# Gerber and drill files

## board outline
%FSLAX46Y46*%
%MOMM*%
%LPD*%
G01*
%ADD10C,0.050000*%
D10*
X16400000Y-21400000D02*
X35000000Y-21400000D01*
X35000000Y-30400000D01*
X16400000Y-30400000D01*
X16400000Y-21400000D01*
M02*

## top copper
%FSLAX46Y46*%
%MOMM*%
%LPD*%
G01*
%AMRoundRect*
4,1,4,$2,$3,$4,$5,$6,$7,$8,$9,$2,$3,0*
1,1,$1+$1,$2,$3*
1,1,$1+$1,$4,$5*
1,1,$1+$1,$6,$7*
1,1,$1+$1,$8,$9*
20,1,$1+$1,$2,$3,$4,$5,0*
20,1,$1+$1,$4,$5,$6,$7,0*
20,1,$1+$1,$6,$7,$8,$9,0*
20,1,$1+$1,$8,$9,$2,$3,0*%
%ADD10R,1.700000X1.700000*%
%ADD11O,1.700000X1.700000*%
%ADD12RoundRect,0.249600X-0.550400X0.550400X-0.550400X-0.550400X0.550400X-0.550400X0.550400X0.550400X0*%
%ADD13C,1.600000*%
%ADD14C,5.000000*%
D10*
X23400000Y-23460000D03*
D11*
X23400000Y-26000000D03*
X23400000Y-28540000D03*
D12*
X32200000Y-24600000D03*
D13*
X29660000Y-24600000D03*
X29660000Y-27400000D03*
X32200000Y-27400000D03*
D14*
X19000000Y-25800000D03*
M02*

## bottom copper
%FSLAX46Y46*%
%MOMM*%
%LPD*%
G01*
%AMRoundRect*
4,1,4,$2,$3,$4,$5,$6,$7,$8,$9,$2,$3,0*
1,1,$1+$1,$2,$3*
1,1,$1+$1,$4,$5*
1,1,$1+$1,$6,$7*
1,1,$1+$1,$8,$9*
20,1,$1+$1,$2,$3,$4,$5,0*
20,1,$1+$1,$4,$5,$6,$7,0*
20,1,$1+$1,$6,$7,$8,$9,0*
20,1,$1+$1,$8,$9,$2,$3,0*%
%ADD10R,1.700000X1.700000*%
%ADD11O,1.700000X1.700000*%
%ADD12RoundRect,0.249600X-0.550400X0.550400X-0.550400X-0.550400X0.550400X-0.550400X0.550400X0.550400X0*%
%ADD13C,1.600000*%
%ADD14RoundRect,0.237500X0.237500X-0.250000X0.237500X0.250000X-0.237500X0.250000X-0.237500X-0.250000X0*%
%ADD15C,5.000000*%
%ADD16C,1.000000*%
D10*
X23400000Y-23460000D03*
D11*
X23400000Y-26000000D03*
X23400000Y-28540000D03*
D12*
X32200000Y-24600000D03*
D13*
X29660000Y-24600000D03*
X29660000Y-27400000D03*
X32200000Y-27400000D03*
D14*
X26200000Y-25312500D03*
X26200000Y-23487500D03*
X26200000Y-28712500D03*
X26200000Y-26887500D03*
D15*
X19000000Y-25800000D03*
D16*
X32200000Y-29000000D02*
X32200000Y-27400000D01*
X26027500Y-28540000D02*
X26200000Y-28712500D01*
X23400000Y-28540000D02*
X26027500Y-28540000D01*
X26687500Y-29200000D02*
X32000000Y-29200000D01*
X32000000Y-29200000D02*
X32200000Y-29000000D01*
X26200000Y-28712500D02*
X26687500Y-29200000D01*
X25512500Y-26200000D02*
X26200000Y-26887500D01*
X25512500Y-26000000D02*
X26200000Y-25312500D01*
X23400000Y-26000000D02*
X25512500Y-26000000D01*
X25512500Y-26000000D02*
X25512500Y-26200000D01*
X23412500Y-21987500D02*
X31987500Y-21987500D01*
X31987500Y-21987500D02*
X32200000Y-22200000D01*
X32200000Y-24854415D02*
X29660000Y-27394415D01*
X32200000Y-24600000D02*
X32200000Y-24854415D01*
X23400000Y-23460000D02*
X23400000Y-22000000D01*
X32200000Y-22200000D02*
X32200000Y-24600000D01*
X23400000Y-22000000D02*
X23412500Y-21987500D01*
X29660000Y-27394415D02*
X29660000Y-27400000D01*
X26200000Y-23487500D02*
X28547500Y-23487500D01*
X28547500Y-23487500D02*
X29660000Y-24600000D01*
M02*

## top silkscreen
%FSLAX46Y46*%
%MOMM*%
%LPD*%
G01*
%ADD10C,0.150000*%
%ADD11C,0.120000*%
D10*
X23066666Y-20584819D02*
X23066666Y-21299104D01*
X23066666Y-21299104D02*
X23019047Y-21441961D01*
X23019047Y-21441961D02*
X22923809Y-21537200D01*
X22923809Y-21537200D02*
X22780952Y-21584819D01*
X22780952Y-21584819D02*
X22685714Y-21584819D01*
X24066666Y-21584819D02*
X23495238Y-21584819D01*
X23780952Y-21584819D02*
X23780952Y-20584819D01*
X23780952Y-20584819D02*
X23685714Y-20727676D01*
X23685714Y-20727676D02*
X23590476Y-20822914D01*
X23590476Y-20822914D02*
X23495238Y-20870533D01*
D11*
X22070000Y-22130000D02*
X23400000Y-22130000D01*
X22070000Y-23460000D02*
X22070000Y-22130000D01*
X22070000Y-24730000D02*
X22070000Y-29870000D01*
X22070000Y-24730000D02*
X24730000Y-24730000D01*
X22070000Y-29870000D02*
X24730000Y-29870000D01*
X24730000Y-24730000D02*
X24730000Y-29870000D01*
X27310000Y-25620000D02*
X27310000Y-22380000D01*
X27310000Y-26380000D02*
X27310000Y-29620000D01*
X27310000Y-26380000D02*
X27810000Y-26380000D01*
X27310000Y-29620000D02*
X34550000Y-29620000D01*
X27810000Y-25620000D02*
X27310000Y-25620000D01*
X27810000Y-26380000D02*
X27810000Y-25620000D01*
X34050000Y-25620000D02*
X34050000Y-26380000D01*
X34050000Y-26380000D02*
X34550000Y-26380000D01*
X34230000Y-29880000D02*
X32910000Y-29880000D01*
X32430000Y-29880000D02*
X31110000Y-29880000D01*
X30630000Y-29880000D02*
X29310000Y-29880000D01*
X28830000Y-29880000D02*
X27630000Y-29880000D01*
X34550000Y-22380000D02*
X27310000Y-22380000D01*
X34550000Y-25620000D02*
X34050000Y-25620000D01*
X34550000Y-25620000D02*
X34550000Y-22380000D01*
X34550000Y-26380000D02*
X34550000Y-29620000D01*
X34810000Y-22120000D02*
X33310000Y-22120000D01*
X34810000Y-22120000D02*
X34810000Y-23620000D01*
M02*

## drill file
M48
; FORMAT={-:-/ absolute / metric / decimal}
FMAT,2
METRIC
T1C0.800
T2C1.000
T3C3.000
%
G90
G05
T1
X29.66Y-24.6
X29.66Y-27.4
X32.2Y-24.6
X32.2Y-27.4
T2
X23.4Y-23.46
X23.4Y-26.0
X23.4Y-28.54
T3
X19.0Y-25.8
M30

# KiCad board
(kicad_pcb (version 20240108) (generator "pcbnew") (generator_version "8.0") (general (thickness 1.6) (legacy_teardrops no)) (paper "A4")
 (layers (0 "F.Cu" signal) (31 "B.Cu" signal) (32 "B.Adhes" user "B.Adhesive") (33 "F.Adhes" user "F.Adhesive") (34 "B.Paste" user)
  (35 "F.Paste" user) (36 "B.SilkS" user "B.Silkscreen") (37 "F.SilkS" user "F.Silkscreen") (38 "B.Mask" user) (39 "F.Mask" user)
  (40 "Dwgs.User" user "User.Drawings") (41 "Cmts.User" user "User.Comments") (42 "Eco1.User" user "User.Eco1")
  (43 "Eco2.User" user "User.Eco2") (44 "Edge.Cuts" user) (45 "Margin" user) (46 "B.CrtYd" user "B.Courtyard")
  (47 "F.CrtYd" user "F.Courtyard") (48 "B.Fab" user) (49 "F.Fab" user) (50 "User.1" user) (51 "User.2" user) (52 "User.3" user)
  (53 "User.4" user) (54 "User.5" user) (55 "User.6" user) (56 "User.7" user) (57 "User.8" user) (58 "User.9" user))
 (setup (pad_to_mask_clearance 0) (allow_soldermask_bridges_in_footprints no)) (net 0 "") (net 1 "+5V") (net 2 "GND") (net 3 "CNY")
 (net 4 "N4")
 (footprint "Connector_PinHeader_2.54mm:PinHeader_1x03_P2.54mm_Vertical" (layer "F.Cu") (at 23.4 23.46)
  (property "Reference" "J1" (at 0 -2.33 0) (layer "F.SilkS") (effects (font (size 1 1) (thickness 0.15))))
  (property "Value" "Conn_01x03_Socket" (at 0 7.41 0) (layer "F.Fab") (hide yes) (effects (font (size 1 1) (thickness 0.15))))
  (fp_line (start -1.33 -1.33) (end 0 -1.33) (stroke (width 0.12) (type solid)) (layer "F.SilkS"))
  (fp_line (start -1.33 0) (end -1.33 -1.33) (stroke (width 0.12) (type solid)) (layer "F.SilkS"))
  (fp_line (start -1.33 1.27) (end -1.33 6.41) (stroke (width 0.12) (type solid)) (layer "F.SilkS"))
  (fp_line (start -1.33 1.27) (end 1.33 1.27) (stroke (width 0.12) (type solid)) (layer "F.SilkS"))
  (fp_line (start -1.33 6.41) (end 1.33 6.41) (stroke (width 0.12) (type solid)) (layer "F.SilkS"))
  (fp_line (start 1.33 1.27) (end 1.33 6.41) (stroke (width 0.12) (type solid)) (layer "F.SilkS"))
  (pad "1" thru_hole rect (at 0 0) (size 1.7 1.7) (drill 1) (layers "*.Cu" "*.Mask") (remove_unused_layers no) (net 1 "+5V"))
  (pad "2" thru_hole oval (at 0 2.54) (size 1.7 1.7) (drill 1) (layers "*.Cu" "*.Mask") (remove_unused_layers no) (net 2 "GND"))
  (pad "3" thru_hole oval (at 0 5.08) (size 1.7 1.7) (drill 1) (layers "*.Cu" "*.Mask") (remove_unused_layers no) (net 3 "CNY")))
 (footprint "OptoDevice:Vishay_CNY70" (layer "F.Cu") (at 32.2 24.6 -90)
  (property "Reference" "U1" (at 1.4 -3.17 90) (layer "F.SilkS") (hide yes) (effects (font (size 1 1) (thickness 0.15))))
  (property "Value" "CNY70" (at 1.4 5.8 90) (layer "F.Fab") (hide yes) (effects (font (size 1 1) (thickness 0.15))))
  (fp_line (start 1.02 4.89) (end -2.22 4.89) (stroke (width 0.12) (type default)) (layer "F.SilkS"))
  (fp_line (start 1.78 4.89) (end 5.02 4.89) (stroke (width 0.12) (type solid)) (layer "F.SilkS"))
  (fp_line (start 1.78 4.89) (end 1.78 4.39) (stroke (width 0.12) (type default)) (layer "F.SilkS"))
  (fp_line (start 5.02 4.89) (end 5.02 -2.35) (stroke (width 0.12) (type solid)) (layer "F.SilkS"))
  (fp_line (start 1.02 4.39) (end 1.02 4.89) (stroke (width 0.12) (type default)) (layer "F.SilkS"))
  (fp_line (start 1.78 4.39) (end 1.02 4.39) (stroke (width 0.12) (type default)) (layer "F.SilkS"))
  (fp_line (start 1.02 -1.85) (end 1.78 -1.85) (stroke (width 0.12) (type default)) (layer "F.SilkS"))
  (fp_line (start 1.78 -1.85) (end 1.78 -2.35) (stroke (width 0.12) (type default)) (layer "F.SilkS"))
  (fp_line (start 5.28 -2.03) (end 5.28 4.57) (stroke (width 0.12) (type dash)) (layer "F.SilkS"))
  (fp_line (start -2.22 -2.35) (end -2.22 4.89) (stroke (width 0.12) (type solid)) (layer "F.SilkS"))
  (fp_line (start 1.02 -2.35) (end 1.02 -1.85) (stroke (width 0.12) (type default)) (layer "F.SilkS"))
  (fp_line (start 1.02 -2.35) (end -2.22 -2.35) (stroke (width 0.12) (type solid)) (layer "F.SilkS"))
  (fp_line (start 1.78 -2.35) (end 5.02 -2.35) (stroke (width 0.12) (type default)) (layer "F.SilkS"))
  (fp_line (start -2.48 -2.61) (end -2.48 -1.11) (stroke (width 0.12) (type default)) (layer "F.SilkS"))
  (fp_line (start -2.48 -2.61) (end -0.98 -2.61) (stroke (width 0.12) (type default)) (layer "F.SilkS"))
  (pad "1" thru_hole roundrect (at 0 0 270) (size 1.6 1.6) (drill 0.8) (layers "*.Cu" "*.Mask") (remove_unused_layers no)
   (roundrect_rratio 0.156) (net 1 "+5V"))
  (pad "2" thru_hole circle (at 0 2.54 270) (size 1.6 1.6) (drill 0.8) (layers "*.Cu" "*.Mask") (remove_unused_layers no) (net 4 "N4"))
  (pad "3" thru_hole circle (at 2.8 2.54 270) (size 1.6 1.6) (drill 0.8) (layers "*.Cu" "*.Mask") (remove_unused_layers no) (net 1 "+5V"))
  (pad "4" thru_hole circle (at 2.8 0 270) (size 1.6 1.6) (drill 0.8) (layers "*.Cu" "*.Mask") (remove_unused_layers no) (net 3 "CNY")))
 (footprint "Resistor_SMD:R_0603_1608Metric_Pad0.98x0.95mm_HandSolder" (layer "B.Cu") (at 26.2 24.4 90)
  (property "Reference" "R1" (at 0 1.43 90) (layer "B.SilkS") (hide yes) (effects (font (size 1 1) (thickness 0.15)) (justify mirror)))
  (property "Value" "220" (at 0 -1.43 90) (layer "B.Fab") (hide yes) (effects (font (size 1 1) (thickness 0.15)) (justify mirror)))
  (pad "1" smd roundrect (at -0.9125 0 90) (size 0.975 0.95) (layers "B.Cu" "B.Paste" "B.Mask") (roundrect_rratio 0.25) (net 2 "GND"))
  (pad "2" smd roundrect (at 0.9125 0 90) (size 0.975 0.95) (layers "B.Cu" "B.Paste" "B.Mask") (roundrect_rratio 0.25) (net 4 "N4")))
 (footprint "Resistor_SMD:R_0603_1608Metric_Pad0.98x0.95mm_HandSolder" (layer "B.Cu") (at 26.2 27.8 90)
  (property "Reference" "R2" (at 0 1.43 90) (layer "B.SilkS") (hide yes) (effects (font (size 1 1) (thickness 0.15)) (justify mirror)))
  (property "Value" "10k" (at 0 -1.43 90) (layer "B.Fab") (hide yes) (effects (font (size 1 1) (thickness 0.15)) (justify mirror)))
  (pad "1" smd roundrect (at -0.9125 0 90) (size 0.975 0.95) (layers "B.Cu" "B.Paste" "B.Mask") (roundrect_rratio 0.25) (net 3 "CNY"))
  (pad "2" smd roundrect (at 0.9125 0 90) (size 0.975 0.95) (layers "B.Cu" "B.Paste" "B.Mask") (roundrect_rratio 0.25) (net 2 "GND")))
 (gr_rect (start 16.4 21.4) (end 35 30.4) (stroke (width 0.05) (type default)) (fill none) (layer "Edge.Cuts"))
 (via (at 19 25.8) (size 5) (drill 3) (layers "F.Cu" "B.Cu") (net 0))
 (segment (start 32.2 29) (end 32.2 27.4) (width 1) (layer "B.Cu") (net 3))
 (segment (start 26.0275 28.54) (end 26.2 28.7125) (width 1) (layer "B.Cu") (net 3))
 (segment (start 23.4 28.54) (end 26.0275 28.54) (width 1) (layer "B.Cu") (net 3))
 (segment (start 26.6875 29.2) (end 32 29.2) (width 1) (layer "B.Cu") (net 3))
 (segment (start 32 29.2) (end 32.2 29) (width 1) (layer "B.Cu") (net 3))
 (segment (start 26.2 28.7125) (end 26.6875 29.2) (width 1) (layer "B.Cu") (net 3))
 (segment (start 25.5125 26.2) (end 26.2 26.8875) (width 1) (layer "B.Cu") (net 2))
 (segment (start 25.5125 26) (end 26.2 25.3125) (width 1) (layer "B.Cu") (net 2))
 (segment (start 23.4 26) (end 25.5125 26) (width 1) (layer "B.Cu") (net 2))
 (segment (start 25.5125 26) (end 25.5125 26.2) (width 1) (layer "B.Cu") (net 2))
 (segment (start 23.4125 21.9875) (end 31.9875 21.9875) (width 1) (layer "B.Cu") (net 1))
 (segment (start 31.9875 21.9875) (end 32.2 22.2) (width 1) (layer "B.Cu") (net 1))
 (segment (start 32.2 24.854415) (end 29.66 27.394415) (width 1) (layer "B.Cu") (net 1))
 (segment (start 32.2 24.6) (end 32.2 24.854415) (width 1) (layer "B.Cu") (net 1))
 (segment (start 23.4 23.46) (end 23.4 22) (width 1) (layer "B.Cu") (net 1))
 (segment (start 32.2 22.2) (end 32.2 24.6) (width 1) (layer "B.Cu") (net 1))
 (segment (start 23.4 22) (end 23.4125 21.9875) (width 1) (layer "B.Cu") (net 1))
 (segment (start 29.66 27.394415) (end 29.66 27.4) (width 1) (layer "B.Cu") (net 1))
 (segment (start 26.2 23.4875) (end 28.5475 23.4875) (width 1) (layer "B.Cu") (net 4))
 (segment (start 28.5475 23.4875) (end 29.66 24.6) (width 1) (layer "B.Cu") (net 4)))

